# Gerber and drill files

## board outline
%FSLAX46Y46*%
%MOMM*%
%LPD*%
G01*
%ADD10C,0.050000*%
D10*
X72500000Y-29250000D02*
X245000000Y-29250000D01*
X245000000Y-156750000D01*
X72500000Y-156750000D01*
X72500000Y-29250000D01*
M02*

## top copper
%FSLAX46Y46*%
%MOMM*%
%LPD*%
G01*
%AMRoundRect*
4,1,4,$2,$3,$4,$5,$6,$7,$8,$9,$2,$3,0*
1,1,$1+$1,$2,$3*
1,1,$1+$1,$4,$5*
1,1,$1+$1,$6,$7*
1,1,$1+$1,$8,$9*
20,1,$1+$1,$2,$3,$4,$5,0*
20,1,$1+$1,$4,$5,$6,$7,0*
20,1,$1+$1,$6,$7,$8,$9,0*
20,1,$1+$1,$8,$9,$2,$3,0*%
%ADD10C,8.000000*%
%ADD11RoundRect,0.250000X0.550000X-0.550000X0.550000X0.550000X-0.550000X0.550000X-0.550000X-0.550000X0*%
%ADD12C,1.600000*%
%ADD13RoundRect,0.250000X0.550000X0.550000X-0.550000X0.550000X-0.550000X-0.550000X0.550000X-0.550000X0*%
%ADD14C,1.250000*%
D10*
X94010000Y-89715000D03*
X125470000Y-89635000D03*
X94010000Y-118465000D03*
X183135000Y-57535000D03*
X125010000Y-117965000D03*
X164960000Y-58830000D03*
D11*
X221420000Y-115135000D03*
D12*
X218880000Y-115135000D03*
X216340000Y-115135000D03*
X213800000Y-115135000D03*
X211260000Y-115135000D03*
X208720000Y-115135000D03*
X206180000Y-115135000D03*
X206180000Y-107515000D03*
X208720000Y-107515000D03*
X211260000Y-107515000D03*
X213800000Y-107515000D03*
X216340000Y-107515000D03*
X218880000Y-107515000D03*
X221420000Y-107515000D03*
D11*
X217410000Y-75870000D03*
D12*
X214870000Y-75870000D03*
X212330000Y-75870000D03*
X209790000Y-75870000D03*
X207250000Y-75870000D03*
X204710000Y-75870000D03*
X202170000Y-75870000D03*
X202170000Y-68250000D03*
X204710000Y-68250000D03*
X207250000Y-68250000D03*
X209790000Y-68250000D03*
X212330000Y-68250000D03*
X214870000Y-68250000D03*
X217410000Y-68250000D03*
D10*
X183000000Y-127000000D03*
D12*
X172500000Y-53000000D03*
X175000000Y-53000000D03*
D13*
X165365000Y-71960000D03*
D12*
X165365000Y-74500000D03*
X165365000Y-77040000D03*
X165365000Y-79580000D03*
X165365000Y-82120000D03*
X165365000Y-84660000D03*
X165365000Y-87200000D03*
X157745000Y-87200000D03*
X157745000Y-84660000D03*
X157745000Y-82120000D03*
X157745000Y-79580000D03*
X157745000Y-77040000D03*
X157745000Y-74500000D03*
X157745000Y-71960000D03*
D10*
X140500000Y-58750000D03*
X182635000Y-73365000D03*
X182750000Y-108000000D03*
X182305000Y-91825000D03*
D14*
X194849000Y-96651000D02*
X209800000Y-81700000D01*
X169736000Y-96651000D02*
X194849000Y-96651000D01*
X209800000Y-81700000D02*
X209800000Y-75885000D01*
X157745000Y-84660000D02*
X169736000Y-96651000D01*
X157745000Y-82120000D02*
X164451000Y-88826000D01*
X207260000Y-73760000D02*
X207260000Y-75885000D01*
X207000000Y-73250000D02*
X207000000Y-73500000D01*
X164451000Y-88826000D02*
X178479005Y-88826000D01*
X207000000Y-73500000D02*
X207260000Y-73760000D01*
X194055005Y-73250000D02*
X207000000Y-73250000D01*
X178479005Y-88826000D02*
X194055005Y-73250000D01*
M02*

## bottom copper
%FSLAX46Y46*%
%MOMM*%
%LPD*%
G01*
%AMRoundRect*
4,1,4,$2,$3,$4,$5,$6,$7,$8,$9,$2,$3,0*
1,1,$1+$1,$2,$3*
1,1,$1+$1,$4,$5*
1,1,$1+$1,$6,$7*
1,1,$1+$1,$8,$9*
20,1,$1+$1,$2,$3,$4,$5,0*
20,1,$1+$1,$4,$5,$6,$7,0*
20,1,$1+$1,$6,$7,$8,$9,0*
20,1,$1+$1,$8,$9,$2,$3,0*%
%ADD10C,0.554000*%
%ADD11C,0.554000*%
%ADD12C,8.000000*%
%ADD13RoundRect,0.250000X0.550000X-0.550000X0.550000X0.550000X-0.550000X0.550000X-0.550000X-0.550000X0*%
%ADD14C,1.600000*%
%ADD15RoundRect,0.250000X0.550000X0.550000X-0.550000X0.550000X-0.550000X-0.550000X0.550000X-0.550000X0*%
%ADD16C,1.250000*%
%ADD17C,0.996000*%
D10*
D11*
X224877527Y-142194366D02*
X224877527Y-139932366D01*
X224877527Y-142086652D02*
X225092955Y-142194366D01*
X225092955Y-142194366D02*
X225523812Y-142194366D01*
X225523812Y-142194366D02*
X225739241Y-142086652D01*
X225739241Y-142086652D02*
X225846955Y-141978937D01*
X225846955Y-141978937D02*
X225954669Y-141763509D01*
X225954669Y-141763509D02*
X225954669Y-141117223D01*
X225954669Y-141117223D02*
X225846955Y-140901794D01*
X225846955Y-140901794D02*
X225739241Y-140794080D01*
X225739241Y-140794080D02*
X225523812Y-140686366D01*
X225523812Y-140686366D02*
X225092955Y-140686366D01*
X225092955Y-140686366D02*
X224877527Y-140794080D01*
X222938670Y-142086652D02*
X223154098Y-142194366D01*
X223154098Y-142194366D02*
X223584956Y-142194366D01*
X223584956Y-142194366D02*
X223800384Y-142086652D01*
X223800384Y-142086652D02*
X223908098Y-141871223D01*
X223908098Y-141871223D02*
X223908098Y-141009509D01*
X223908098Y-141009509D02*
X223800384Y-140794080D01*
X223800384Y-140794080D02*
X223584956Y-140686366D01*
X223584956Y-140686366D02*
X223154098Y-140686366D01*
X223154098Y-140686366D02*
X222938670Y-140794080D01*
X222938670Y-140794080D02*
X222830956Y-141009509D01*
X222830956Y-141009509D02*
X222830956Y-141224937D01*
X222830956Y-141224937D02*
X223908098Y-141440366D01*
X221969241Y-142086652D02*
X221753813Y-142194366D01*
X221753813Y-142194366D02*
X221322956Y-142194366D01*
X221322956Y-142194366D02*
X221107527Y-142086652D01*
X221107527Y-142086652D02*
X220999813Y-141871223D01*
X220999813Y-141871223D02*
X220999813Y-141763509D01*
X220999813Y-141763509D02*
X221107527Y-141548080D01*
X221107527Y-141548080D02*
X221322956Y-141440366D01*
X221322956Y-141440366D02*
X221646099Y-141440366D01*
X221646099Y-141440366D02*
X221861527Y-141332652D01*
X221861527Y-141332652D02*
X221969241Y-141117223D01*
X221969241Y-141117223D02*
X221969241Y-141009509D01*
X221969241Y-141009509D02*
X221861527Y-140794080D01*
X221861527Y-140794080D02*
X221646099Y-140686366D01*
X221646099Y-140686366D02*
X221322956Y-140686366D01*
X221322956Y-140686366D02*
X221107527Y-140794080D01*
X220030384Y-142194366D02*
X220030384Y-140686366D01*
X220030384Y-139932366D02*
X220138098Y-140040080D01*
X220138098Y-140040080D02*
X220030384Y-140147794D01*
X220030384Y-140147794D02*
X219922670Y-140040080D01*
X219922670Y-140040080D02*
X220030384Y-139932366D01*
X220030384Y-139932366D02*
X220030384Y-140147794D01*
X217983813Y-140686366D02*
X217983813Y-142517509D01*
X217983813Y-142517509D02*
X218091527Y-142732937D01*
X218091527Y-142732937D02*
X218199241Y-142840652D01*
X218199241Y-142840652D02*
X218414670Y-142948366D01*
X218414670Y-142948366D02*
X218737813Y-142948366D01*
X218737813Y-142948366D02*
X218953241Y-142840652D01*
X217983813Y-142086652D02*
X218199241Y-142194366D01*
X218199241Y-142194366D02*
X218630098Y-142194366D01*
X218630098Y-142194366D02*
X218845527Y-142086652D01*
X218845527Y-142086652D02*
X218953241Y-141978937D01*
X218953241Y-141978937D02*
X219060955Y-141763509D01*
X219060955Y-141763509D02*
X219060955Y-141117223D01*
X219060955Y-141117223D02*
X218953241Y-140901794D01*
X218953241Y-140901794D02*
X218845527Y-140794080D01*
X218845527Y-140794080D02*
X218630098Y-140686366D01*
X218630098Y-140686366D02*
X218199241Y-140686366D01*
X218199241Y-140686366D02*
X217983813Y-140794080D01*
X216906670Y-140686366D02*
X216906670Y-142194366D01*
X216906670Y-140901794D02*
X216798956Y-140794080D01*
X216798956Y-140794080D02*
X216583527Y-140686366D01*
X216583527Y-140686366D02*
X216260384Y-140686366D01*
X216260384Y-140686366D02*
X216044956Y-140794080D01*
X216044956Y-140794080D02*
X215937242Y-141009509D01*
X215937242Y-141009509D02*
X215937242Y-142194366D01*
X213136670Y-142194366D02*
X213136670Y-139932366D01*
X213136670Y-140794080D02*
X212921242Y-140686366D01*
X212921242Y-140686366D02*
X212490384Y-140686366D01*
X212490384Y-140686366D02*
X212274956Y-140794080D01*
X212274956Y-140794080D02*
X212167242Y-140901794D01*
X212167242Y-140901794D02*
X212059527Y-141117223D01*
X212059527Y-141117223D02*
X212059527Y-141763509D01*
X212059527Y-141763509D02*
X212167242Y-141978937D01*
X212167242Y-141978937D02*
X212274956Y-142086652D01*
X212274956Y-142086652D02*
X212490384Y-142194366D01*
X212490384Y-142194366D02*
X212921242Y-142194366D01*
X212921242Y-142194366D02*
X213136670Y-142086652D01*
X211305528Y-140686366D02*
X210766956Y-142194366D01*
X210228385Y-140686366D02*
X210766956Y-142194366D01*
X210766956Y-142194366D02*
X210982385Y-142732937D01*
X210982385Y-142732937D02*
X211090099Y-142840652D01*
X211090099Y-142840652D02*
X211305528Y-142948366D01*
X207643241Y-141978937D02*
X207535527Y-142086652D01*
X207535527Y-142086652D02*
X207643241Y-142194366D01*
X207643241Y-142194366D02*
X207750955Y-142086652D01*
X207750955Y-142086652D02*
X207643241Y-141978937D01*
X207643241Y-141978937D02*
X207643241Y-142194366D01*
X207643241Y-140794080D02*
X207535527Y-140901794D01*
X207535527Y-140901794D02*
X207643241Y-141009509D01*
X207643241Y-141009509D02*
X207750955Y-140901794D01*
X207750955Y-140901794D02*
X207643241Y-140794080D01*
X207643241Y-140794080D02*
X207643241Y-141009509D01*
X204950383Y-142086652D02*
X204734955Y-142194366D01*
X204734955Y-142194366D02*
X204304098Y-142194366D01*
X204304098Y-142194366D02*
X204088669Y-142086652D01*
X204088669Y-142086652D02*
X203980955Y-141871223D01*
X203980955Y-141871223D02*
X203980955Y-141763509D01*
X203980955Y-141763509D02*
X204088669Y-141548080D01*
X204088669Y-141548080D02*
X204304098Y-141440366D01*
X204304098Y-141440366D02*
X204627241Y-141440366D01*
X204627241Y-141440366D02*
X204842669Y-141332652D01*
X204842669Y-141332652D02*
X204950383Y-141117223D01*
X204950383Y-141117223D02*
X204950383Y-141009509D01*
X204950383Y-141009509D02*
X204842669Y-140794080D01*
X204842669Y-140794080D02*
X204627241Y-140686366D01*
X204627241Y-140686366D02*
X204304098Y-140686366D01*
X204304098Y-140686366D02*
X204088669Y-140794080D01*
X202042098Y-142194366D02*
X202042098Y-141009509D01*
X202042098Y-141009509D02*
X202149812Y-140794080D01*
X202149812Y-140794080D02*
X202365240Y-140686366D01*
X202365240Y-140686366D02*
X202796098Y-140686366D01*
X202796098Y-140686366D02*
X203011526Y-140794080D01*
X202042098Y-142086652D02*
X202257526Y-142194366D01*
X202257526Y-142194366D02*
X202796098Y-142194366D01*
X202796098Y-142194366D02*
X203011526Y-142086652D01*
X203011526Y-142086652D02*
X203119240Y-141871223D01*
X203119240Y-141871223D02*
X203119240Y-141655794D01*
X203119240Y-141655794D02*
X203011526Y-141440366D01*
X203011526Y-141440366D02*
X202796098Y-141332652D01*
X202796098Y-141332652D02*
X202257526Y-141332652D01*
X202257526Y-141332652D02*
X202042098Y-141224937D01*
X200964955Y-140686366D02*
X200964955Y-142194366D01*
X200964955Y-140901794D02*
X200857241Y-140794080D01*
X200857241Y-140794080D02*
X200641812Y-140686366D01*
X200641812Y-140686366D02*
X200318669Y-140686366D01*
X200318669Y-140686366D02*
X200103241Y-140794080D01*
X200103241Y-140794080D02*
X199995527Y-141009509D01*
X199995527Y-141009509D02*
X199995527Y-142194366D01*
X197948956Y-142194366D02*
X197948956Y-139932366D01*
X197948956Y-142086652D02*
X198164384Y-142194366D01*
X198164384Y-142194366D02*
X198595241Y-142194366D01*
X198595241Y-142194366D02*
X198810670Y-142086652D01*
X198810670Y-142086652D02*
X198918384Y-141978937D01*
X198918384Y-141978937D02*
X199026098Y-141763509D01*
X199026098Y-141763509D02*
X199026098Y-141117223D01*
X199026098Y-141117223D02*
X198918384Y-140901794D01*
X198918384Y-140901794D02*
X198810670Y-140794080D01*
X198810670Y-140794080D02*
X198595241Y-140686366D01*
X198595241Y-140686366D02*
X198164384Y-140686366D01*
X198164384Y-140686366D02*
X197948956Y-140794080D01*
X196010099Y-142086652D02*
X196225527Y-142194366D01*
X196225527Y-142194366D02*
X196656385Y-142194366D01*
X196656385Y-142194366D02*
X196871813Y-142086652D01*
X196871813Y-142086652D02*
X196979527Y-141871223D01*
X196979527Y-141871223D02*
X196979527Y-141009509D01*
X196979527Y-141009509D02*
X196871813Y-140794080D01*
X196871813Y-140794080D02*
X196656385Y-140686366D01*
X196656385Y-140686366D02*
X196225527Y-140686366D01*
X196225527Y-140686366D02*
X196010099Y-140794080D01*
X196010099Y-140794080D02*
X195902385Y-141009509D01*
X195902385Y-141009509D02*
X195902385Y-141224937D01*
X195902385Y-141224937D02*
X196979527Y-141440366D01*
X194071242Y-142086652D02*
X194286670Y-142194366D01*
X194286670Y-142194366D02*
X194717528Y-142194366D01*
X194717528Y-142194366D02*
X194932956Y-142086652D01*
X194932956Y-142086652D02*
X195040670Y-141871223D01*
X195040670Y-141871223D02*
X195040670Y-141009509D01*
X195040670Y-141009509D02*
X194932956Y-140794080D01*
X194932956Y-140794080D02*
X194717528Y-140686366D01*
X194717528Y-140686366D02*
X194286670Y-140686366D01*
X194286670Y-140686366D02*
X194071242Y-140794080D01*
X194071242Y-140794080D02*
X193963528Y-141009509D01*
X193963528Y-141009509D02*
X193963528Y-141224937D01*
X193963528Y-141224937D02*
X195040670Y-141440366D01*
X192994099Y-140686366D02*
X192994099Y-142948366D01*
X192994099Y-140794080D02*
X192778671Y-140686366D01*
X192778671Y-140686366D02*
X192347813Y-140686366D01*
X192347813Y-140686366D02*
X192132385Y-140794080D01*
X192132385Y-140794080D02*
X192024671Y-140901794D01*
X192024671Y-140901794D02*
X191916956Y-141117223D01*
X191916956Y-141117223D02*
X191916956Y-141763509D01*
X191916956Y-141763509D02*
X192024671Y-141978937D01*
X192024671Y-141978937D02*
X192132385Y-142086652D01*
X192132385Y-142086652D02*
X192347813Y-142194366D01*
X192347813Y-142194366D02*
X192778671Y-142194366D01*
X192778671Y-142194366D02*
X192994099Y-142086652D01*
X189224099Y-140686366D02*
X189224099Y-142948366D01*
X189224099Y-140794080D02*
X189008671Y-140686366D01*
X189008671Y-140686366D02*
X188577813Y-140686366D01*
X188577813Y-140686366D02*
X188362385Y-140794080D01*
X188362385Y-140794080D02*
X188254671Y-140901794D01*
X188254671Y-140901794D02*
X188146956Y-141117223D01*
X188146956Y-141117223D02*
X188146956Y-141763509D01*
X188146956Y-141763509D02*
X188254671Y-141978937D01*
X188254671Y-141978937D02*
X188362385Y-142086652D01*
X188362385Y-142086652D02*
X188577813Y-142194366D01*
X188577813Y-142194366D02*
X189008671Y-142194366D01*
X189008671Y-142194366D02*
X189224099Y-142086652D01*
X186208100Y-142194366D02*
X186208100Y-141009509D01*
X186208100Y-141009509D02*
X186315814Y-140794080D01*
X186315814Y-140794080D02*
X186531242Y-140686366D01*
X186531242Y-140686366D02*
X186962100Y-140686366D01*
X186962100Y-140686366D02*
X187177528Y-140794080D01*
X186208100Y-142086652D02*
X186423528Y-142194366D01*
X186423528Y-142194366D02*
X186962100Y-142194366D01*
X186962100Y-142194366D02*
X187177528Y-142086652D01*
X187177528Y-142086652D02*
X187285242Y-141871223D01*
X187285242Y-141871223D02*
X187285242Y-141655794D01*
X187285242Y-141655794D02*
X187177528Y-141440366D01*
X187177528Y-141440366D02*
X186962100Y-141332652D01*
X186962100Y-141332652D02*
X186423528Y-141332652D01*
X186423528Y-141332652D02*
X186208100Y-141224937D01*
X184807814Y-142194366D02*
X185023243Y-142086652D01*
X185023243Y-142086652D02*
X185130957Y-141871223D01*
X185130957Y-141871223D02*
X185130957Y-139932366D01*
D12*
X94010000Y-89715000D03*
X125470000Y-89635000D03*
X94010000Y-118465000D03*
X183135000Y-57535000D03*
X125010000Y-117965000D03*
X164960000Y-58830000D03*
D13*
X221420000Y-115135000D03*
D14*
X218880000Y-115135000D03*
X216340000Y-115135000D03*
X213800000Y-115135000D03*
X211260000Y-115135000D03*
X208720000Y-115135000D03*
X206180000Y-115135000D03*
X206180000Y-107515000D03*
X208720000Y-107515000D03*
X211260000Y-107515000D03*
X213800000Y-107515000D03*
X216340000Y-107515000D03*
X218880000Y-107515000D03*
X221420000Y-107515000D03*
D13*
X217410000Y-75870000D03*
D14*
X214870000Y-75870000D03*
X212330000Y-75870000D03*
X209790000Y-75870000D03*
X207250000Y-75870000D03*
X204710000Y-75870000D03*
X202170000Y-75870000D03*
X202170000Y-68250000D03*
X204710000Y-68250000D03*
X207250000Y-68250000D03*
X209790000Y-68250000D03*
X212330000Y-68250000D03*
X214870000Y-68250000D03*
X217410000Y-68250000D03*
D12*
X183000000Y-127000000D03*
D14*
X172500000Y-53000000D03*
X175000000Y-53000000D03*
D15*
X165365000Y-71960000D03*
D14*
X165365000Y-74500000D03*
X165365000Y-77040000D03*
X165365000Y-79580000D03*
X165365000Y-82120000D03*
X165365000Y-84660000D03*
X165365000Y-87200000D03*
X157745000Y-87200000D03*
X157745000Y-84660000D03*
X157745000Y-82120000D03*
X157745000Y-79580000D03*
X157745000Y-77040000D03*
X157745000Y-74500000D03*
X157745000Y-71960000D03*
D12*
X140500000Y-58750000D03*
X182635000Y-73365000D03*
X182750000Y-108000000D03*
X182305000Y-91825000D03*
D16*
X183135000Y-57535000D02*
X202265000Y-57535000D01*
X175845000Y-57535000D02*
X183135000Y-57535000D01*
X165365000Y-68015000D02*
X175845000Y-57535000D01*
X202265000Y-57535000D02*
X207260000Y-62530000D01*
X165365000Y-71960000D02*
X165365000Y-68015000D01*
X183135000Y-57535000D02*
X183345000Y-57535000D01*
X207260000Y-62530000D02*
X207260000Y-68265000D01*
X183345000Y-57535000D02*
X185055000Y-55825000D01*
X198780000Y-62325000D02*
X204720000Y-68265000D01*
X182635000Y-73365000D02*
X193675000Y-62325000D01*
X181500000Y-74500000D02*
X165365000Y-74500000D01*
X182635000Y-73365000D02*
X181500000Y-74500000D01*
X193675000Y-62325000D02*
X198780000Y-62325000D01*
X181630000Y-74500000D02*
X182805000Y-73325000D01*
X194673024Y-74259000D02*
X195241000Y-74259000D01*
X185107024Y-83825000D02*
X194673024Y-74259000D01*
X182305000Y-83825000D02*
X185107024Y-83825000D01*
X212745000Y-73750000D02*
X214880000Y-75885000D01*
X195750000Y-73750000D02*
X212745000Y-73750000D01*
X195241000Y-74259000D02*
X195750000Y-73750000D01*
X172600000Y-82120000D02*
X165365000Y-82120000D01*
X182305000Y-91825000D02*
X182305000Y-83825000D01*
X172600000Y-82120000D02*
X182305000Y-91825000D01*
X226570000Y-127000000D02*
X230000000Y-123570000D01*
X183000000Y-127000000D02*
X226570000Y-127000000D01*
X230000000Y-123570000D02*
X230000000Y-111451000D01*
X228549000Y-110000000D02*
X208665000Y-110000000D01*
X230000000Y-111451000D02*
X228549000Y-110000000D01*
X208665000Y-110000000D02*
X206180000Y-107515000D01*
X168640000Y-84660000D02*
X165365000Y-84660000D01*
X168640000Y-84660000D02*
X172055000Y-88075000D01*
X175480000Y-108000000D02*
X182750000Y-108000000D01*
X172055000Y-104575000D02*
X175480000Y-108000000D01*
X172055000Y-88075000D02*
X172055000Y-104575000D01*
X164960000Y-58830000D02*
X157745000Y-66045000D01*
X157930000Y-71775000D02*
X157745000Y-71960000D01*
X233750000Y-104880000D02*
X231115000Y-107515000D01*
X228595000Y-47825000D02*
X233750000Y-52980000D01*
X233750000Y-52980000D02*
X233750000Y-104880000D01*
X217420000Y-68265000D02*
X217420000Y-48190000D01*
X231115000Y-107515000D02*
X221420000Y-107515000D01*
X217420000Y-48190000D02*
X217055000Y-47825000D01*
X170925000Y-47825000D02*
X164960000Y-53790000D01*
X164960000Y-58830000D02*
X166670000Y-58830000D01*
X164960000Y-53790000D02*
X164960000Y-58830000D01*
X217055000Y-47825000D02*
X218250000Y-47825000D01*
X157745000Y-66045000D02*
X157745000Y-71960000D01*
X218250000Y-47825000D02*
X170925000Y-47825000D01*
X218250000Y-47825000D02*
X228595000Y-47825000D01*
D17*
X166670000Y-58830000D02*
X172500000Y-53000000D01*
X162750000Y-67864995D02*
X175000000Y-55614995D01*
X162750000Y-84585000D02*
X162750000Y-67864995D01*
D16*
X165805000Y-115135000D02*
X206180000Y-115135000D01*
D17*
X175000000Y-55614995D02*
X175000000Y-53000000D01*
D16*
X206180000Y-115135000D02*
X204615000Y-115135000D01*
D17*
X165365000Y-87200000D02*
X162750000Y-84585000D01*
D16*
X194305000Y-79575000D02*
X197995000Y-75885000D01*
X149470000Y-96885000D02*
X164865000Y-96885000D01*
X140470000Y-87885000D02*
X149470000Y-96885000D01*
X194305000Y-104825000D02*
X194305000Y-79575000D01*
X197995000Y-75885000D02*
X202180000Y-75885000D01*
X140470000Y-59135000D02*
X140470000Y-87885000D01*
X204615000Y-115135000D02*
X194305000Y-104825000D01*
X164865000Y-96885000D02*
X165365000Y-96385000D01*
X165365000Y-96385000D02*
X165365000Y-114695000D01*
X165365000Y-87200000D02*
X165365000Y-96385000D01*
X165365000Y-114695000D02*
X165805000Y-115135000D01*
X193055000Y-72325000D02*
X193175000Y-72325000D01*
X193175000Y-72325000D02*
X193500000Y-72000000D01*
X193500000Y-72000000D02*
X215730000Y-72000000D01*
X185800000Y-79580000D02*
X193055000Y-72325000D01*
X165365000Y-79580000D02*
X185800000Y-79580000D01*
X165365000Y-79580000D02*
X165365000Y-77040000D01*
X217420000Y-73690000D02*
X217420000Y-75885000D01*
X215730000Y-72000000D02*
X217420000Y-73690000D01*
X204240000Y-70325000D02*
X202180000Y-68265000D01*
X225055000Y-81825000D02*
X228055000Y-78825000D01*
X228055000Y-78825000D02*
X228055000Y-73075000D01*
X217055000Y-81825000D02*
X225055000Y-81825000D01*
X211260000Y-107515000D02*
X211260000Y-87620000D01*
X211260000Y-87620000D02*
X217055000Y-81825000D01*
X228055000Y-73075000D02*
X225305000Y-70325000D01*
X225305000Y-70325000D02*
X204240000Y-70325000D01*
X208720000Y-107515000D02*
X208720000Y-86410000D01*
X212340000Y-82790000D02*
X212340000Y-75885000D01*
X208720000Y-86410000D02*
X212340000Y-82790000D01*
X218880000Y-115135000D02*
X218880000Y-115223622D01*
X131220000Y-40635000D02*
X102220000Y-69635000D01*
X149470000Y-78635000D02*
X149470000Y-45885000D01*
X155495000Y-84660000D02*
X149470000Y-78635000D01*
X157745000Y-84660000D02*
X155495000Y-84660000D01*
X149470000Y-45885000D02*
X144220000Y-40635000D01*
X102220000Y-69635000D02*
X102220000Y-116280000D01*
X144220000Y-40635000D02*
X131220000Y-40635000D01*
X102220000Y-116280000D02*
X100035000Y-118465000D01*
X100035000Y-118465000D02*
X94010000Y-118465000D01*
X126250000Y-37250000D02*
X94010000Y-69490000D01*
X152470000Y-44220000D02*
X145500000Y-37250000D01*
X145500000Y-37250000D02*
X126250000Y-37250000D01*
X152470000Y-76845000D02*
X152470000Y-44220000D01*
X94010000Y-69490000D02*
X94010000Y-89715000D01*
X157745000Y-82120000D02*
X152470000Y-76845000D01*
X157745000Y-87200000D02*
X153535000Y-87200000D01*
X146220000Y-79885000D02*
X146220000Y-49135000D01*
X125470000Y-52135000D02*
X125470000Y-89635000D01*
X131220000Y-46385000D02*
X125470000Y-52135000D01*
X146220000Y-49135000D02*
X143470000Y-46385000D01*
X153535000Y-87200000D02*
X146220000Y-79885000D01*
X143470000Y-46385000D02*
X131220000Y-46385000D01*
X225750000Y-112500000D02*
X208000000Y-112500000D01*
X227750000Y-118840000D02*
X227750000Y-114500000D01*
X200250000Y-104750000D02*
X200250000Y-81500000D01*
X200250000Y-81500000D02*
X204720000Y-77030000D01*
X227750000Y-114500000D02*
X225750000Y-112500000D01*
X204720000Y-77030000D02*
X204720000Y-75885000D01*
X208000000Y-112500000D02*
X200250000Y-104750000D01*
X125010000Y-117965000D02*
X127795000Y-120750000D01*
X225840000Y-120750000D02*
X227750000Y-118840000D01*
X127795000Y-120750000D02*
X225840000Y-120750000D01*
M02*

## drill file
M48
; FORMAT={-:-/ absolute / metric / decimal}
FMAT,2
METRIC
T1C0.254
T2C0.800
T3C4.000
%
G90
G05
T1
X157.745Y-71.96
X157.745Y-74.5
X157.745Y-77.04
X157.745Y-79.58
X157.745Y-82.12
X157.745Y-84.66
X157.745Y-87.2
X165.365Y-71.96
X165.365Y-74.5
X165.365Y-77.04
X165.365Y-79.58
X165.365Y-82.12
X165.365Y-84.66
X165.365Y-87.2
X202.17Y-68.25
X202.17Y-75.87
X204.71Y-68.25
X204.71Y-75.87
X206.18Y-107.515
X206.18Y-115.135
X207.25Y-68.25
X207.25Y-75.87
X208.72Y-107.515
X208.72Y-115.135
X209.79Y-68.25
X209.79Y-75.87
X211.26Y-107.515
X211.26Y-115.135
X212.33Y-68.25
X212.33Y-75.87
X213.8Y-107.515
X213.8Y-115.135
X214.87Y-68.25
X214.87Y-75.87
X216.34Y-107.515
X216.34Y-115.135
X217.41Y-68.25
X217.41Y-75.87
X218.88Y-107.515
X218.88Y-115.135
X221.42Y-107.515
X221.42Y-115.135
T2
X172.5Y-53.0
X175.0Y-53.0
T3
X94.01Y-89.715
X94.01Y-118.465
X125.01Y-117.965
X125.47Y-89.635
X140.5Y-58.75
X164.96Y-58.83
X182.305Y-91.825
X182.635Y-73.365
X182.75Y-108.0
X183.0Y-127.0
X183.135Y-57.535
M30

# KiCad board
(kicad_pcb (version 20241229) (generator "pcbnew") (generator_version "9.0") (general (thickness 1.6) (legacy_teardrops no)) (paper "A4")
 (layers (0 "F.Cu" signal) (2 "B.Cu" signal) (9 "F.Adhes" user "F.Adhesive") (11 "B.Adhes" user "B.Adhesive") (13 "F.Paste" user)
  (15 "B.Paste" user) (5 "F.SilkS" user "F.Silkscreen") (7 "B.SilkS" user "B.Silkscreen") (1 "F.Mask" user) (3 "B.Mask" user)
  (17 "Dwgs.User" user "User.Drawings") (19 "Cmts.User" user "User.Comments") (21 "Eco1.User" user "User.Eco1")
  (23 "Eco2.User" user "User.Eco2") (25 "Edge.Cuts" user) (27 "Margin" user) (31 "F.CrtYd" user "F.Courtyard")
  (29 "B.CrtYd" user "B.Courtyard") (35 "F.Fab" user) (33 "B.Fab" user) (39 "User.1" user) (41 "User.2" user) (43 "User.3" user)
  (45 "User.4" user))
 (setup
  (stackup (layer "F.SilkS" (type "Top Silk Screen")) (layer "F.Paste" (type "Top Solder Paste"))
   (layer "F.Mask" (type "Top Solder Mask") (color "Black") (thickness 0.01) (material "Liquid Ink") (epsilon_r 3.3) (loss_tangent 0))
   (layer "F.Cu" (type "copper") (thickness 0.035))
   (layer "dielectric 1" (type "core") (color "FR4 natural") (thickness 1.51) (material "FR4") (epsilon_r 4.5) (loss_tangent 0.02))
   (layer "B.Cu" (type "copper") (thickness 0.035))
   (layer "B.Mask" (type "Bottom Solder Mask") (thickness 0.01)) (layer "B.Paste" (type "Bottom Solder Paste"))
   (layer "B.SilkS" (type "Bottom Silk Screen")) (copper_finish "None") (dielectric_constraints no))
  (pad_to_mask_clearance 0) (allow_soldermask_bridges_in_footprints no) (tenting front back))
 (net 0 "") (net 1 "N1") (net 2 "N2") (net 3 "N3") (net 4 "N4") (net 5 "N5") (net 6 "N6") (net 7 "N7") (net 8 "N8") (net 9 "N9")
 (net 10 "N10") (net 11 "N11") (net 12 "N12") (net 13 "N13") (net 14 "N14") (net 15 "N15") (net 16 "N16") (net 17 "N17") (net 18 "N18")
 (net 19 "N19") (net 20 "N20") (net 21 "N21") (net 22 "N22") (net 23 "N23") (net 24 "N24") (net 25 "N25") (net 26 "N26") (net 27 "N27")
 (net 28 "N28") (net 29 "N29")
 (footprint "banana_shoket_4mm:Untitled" (layer "F.Cu") (at 94.22 89.635)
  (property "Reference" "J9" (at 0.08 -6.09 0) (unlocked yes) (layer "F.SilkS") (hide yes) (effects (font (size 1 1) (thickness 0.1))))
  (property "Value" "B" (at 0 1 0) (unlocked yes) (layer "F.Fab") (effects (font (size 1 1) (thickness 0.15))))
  (pad "1" thru_hole circle (at -0.21 0.08) (size 8 8) (drill 4) (layers "*.Cu" "*.Mask") (remove_unused_layers no) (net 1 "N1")))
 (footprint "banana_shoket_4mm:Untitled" (layer "F.Cu") (at 125.68 89.555)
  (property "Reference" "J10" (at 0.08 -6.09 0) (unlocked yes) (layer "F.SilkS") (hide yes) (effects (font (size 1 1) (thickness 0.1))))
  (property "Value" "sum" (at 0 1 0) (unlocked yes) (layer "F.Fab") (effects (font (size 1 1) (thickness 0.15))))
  (pad "1" thru_hole circle (at -0.21 0.08) (size 8 8) (drill 4) (layers "*.Cu" "*.Mask") (remove_unused_layers no) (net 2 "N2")))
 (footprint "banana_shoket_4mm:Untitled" (layer "F.Cu") (at 94.22 118.385)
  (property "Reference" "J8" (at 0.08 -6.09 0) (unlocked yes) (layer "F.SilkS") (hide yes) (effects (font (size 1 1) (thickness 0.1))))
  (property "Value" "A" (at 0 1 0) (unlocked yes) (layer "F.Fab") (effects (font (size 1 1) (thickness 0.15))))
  (pad "1" thru_hole circle (at -0.21 0.08) (size 8 8) (drill 4) (layers "*.Cu" "*.Mask") (remove_unused_layers no) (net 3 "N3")))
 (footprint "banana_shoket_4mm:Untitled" (layer "F.Cu") (at 183.055 57.325 90)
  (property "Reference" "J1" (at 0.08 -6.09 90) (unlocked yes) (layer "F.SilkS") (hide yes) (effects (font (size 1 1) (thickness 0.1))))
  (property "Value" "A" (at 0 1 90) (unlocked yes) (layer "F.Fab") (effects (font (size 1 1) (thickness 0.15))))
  (pad "1" thru_hole circle (at -0.21 0.08 90) (size 8 8) (drill 4) (layers "*.Cu" "*.Mask") (remove_unused_layers no) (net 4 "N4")))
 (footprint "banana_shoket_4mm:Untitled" (layer "F.Cu") (at 125.22 117.885)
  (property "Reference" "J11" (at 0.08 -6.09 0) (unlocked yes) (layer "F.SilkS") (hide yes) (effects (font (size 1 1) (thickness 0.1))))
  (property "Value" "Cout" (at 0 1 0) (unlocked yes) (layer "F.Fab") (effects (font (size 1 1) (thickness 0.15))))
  (pad "1" thru_hole circle (at -0.21 0.08) (size 8 8) (drill 4) (layers "*.Cu" "*.Mask") (remove_unused_layers no) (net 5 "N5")))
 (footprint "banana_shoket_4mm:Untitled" (layer "B.Cu") (at 164.75 58.75 180)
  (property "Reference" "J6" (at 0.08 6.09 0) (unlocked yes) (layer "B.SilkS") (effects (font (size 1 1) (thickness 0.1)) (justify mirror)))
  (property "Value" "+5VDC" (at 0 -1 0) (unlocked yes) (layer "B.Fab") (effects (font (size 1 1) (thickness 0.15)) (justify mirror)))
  (pad "1" thru_hole circle (at -0.21 -0.08 180) (size 8 8) (drill 4) (layers "*.Cu" "*.Mask") (remove_unused_layers no) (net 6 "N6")))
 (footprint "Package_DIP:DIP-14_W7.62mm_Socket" (layer "B.Cu") (at 221.42 115.135 90)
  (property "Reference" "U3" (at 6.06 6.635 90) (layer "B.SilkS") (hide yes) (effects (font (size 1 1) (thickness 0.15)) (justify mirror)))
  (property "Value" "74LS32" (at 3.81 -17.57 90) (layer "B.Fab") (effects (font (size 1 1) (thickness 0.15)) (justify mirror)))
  (pad "1" thru_hole roundrect (at 0 0 90) (size 1.6 1.6) (drill 0.254) (layers "*.Cu" "*.Mask") (remove_unused_layers no)
   (roundrect_rratio 0.15625) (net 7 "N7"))
  (pad "2" thru_hole circle (at 0 -2.54 90) (size 1.6 1.6) (drill 0.254) (layers "*.Cu" "*.Mask") (remove_unused_layers no) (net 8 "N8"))
  (pad "3" thru_hole circle (at 0 -5.08 90) (size 1.6 1.6) (drill 0.254) (layers "*.Cu" "*.Mask") (remove_unused_layers no) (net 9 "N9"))
  (pad "4" thru_hole circle (at 0 -7.62 90) (size 1.6 1.6) (drill 0.254) (layers "*.Cu" "*.Mask") (remove_unused_layers no) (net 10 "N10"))
  (pad "5" thru_hole circle (at 0 -10.16 90) (size 1.6 1.6) (drill 0.254) (layers "*.Cu" "*.Mask") (remove_unused_layers no) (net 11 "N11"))
  (pad "6" thru_hole circle (at 0 -12.7 90) (size 1.6 1.6) (drill 0.254) (layers "*.Cu" "*.Mask") (remove_unused_layers no) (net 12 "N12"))
  (pad "7" thru_hole circle (at 0 -15.24 90) (size 1.6 1.6) (drill 0.254) (layers "*.Cu" "*.Mask") (remove_unused_layers no) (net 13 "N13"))
  (pad "8" thru_hole circle (at 7.62 -15.24 90) (size 1.6 1.6) (drill 0.254) (layers "*.Cu" "*.Mask") (remove_unused_layers no)
   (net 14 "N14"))
  (pad "9" thru_hole circle (at 7.62 -12.7 90) (size 1.6 1.6) (drill 0.254) (layers "*.Cu" "*.Mask") (remove_unused_layers no)
   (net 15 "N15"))
  (pad "10" thru_hole circle (at 7.62 -10.16 90) (size 1.6 1.6) (drill 0.254) (layers "*.Cu" "*.Mask") (remove_unused_layers no)
   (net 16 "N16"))
  (pad "11" thru_hole circle (at 7.62 -7.62 90) (size 1.6 1.6) (drill 0.254) (layers "*.Cu" "*.Mask") (remove_unused_layers no)
   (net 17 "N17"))
  (pad "12" thru_hole circle (at 7.62 -5.08 90) (size 1.6 1.6) (drill 0.254) (layers "*.Cu" "*.Mask") (remove_unused_layers no)
   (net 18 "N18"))
  (pad "13" thru_hole circle (at 7.62 -2.54 90) (size 1.6 1.6) (drill 0.254) (layers "*.Cu" "*.Mask") (remove_unused_layers no)
   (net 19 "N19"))
  (pad "14" thru_hole circle (at 7.62 0 90) (size 1.6 1.6) (drill 0.254) (layers "*.Cu" "*.Mask") (remove_unused_layers no) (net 6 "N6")))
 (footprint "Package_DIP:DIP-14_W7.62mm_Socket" (layer "B.Cu") (at 217.41 75.87 90)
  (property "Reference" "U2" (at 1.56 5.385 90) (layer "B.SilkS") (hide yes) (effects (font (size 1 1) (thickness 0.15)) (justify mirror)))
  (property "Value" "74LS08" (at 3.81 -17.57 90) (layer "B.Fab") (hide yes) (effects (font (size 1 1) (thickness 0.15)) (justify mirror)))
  (pad "1" thru_hole roundrect (at 0 0 90) (size 1.6 1.6) (drill 0.254) (layers "*.Cu" "*.Mask") (remove_unused_layers no)
   (roundrect_rratio 0.15625) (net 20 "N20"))
  (pad "2" thru_hole circle (at 0 -2.54 90) (size 1.6 1.6) (drill 0.254) (layers "*.Cu" "*.Mask") (remove_unused_layers no) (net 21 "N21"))
  (pad "3" thru_hole circle (at 0 -5.08 90) (size 1.6 1.6) (drill 0.254) (layers "*.Cu" "*.Mask") (remove_unused_layers no) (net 15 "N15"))
  (pad "4" thru_hole circle (at 0 -7.62 90) (size 1.6 1.6) (drill 0.254) (layers "*.Cu" "*.Mask") (remove_unused_layers no) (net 3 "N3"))
  (pad "5" thru_hole circle (at 0 -10.16 90) (size 1.6 1.6) (drill 0.254) (layers "*.Cu" "*.Mask") (remove_unused_layers no) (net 1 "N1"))
  (pad "6" thru_hole circle (at 0 -12.7 90) (size 1.6 1.6) (drill 0.254) (layers "*.Cu" "*.Mask") (remove_unused_layers no) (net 5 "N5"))
  (pad "7" thru_hole circle (at 0 -15.24 90) (size 1.6 1.6) (drill 0.254) (layers "*.Cu" "*.Mask") (remove_unused_layers no) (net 13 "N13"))
  (pad "8" thru_hole circle (at 7.62 -15.24 90) (size 1.6 1.6) (drill 0.254) (layers "*.Cu" "*.Mask") (remove_unused_layers no)
   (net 16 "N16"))
  (pad "9" thru_hole circle (at 7.62 -12.7 90) (size 1.6 1.6) (drill 0.254) (layers "*.Cu" "*.Mask") (remove_unused_layers no)
   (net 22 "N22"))
  (pad "10" thru_hole circle (at 7.62 -10.16 90) (size 1.6 1.6) (drill 0.254) (layers "*.Cu" "*.Mask") (remove_unused_layers no)
   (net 4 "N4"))
  (pad "11" thru_hole circle (at 7.62 -7.62 90) (size 1.6 1.6) (drill 0.254) (layers "*.Cu" "*.Mask") (remove_unused_layers no)
   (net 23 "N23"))
  (pad "12" thru_hole circle (at 7.62 -5.08 90) (size 1.6 1.6) (drill 0.254) (layers "*.Cu" "*.Mask") (remove_unused_layers no)
   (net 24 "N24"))
  (pad "13" thru_hole circle (at 7.62 -2.54 90) (size 1.6 1.6) (drill 0.254) (layers "*.Cu" "*.Mask") (remove_unused_layers no)
   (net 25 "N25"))
  (pad "14" thru_hole circle (at 7.62 0 90) (size 1.6 1.6) (drill 0.254) (layers "*.Cu" "*.Mask") (remove_unused_layers no) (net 6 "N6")))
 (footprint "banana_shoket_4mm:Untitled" (layer "B.Cu") (at 182.79 126.92 180)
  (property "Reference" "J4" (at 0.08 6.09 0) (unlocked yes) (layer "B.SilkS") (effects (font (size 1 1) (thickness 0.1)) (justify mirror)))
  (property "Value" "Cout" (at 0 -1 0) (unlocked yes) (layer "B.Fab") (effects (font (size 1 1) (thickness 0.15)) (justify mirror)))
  (pad "1" thru_hole circle (at -0.21 -0.08 180) (size 8 8) (drill 4) (layers "*.Cu" "*.Mask") (remove_unused_layers no) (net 14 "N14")))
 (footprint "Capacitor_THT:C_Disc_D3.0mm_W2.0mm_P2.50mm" (layer "B.Cu") (at 172.5 53)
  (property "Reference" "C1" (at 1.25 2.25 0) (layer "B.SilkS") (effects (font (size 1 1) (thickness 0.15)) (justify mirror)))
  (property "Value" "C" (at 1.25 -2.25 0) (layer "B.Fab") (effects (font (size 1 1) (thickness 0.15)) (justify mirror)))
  (pad "1" thru_hole circle (at 0 0) (size 1.6 1.6) (drill 0.8) (layers "*.Cu" "*.Mask") (remove_unused_layers no) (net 6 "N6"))
  (pad "2" thru_hole circle (at 2.5 0) (size 1.6 1.6) (drill 0.8) (layers "*.Cu" "*.Mask") (remove_unused_layers no) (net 13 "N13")))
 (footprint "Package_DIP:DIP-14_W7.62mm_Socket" (layer "B.Cu") (at 165.365 71.96 180)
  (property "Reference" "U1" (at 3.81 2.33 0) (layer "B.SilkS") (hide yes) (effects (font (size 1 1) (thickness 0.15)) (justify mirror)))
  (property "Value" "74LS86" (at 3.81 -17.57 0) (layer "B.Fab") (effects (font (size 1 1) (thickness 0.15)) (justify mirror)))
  (pad "1" thru_hole roundrect (at 0 0 180) (size 1.6 1.6) (drill 0.254) (layers "*.Cu" "*.Mask") (remove_unused_layers no)
   (roundrect_rratio 0.15625) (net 4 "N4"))
  (pad "2" thru_hole circle (at 0 -2.54 180) (size 1.6 1.6) (drill 0.254) (layers "*.Cu" "*.Mask") (remove_unused_layers no) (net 22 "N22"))
  (pad "3" thru_hole circle (at 0 -5.08 180) (size 1.6 1.6) (drill 0.254) (layers "*.Cu" "*.Mask") (remove_unused_layers no) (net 20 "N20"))
  (pad "4" thru_hole circle (at 0 -7.62 180) (size 1.6 1.6) (drill 0.254) (layers "*.Cu" "*.Mask") (remove_unused_layers no) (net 20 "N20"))
  (pad "5" thru_hole circle (at 0 -10.16 180) (size 1.6 1.6) (drill 0.254) (layers "*.Cu" "*.Mask") (remove_unused_layers no) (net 21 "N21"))
  (pad "6" thru_hole circle (at 0 -12.7 180) (size 1.6 1.6) (drill 0.254) (layers "*.Cu" "*.Mask") (remove_unused_layers no) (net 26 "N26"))
  (pad "7" thru_hole circle (at 0 -15.24 180) (size 1.6 1.6) (drill 0.254) (layers "*.Cu" "*.Mask") (remove_unused_layers no) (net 13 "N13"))
  (pad "8" thru_hole circle (at 7.62 -15.24 180) (size 1.6 1.6) (drill 0.254) (layers "*.Cu" "*.Mask") (remove_unused_layers no)
   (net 2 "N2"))
  (pad "9" thru_hole circle (at 7.62 -12.7 180) (size 1.6 1.6) (drill 0.254) (layers "*.Cu" "*.Mask") (remove_unused_layers no) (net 3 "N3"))
  (pad "10" thru_hole circle (at 7.62 -10.16 180) (size 1.6 1.6) (drill 0.254) (layers "*.Cu" "*.Mask") (remove_unused_layers no)
   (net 1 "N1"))
  (pad "11" thru_hole circle (at 7.62 -7.62 180) (size 1.6 1.6) (drill 0.254) (layers "*.Cu" "*.Mask") (remove_unused_layers no)
   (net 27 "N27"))
  (pad "12" thru_hole circle (at 7.62 -5.08 180) (size 1.6 1.6) (drill 0.254) (layers "*.Cu" "*.Mask") (remove_unused_layers no)
   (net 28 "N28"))
  (pad "13" thru_hole circle (at 7.62 -2.54 180) (size 1.6 1.6) (drill 0.254) (layers "*.Cu" "*.Mask") (remove_unused_layers no)
   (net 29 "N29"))
  (pad "14" thru_hole circle (at 7.62 0 180) (size 1.6 1.6) (drill 0.254) (layers "*.Cu" "*.Mask") (remove_unused_layers no) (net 6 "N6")))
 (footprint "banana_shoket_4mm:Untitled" (layer "B.Cu") (at 140.42 58.96 -90)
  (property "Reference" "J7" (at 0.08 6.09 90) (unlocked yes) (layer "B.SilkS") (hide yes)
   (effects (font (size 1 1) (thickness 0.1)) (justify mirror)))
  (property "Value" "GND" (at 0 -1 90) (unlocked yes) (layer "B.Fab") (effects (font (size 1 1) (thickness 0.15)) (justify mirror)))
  (pad "1" thru_hole circle (at -0.21 -0.08 270) (size 8 8) (drill 4) (layers "*.Cu" "*.Mask") (remove_unused_layers no) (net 13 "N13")))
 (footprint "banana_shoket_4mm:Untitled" (layer "B.Cu") (at 182.555 73.575 -90)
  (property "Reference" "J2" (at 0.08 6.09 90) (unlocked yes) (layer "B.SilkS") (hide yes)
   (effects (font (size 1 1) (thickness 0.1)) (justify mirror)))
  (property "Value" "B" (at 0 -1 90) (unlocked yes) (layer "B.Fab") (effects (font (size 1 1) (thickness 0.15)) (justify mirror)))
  (pad "1" thru_hole circle (at -0.21 -0.08 270) (size 8 8) (drill 4) (layers "*.Cu" "*.Mask") (remove_unused_layers no) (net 22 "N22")))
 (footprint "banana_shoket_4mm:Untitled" (layer "B.Cu") (at 182.54 107.92 180)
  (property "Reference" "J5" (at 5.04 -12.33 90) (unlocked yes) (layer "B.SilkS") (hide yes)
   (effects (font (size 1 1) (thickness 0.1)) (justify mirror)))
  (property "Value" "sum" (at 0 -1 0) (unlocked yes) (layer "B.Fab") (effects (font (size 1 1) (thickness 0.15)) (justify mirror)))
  (pad "1" thru_hole circle (at -0.21 -0.08 180) (size 8 8) (drill 4) (layers "*.Cu" "*.Mask") (remove_unused_layers no) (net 26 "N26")))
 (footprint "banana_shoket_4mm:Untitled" (layer "B.Cu") (at 182.225 92.035 -90)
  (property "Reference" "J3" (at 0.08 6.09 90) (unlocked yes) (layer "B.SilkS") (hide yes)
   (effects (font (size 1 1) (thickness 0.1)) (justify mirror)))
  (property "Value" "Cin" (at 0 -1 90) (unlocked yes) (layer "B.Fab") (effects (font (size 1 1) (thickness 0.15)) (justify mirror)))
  (pad "1" thru_hole circle (at -0.21 -0.08 270) (size 8 8) (drill 4) (layers "*.Cu" "*.Mask") (remove_unused_layers no) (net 21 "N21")))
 (gr_rect (start 72.5 29.25) (end 245 156.75) (stroke (width 0.05) (type default)) (fill no) (layer "Edge.Cuts"))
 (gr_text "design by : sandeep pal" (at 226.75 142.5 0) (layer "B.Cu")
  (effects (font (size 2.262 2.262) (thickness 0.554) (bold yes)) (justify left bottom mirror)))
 (segment (start 183.135 57.535) (end 202.265 57.535) (width 1.25) (layer "B.Cu") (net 4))
 (segment (start 175.845 57.535) (end 183.135 57.535) (width 1.25) (layer "B.Cu") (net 4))
 (segment (start 165.365 68.015) (end 175.845 57.535) (width 1.25) (layer "B.Cu") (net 4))
 (segment (start 202.265 57.535) (end 207.26 62.53) (width 1.25) (layer "B.Cu") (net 4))
 (segment (start 165.365 71.96) (end 165.365 68.015) (width 1.25) (layer "B.Cu") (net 4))
 (segment (start 183.135 57.535) (end 183.345 57.535) (width 1.25) (layer "B.Cu") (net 4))
 (segment (start 207.26 62.53) (end 207.26 68.265) (width 1.25) (layer "B.Cu") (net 4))
 (segment (start 183.345 57.535) (end 185.055 55.825) (width 1.25) (layer "B.Cu") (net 4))
 (segment (start 198.78 62.325) (end 204.72 68.265) (width 1.25) (layer "B.Cu") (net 22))
 (segment (start 182.635 73.365) (end 193.675 62.325) (width 1.25) (layer "B.Cu") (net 22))
 (segment (start 181.5 74.5) (end 165.365 74.5) (width 1.25) (layer "B.Cu") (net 22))
 (segment (start 182.635 73.365) (end 181.5 74.5) (width 1.25) (layer "B.Cu") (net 22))
 (segment (start 193.675 62.325) (end 198.78 62.325) (width 1.25) (layer "B.Cu") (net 22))
 (segment (start 181.63 74.5) (end 182.805 73.325) (width 1.25) (layer "B.Cu") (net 22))
 (segment (start 194.673024 74.259) (end 195.241 74.259) (width 1.25) (layer "B.Cu") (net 21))
 (segment (start 185.107024 83.825) (end 194.673024 74.259) (width 1.25) (layer "B.Cu") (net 21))
 (segment (start 182.305 83.825) (end 185.107024 83.825) (width 1.25) (layer "B.Cu") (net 21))
 (segment (start 212.745 73.75) (end 214.88 75.885) (width 1.25) (layer "B.Cu") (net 21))
 (segment (start 195.75 73.75) (end 212.745 73.75) (width 1.25) (layer "B.Cu") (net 21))
 (segment (start 195.241 74.259) (end 195.75 73.75) (width 1.25) (layer "B.Cu") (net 21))
 (segment (start 172.6 82.12) (end 165.365 82.12) (width 1.25) (layer "B.Cu") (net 21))
 (segment (start 182.305 91.825) (end 182.305 83.825) (width 1.25) (layer "B.Cu") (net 21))
 (segment (start 172.6 82.12) (end 182.305 91.825) (width 1.25) (layer "B.Cu") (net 21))
 (segment (start 226.57 127) (end 230 123.57) (width 1.25) (layer "B.Cu") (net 14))
 (segment (start 183 127) (end 226.57 127) (width 1.25) (layer "B.Cu") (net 14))
 (segment (start 230 123.57) (end 230 111.451) (width 1.25) (layer "B.Cu") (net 14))
 (segment (start 228.549 110) (end 208.665 110) (width 1.25) (layer "B.Cu") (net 14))
 (segment (start 230 111.451) (end 228.549 110) (width 1.25) (layer "B.Cu") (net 14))
 (segment (start 208.665 110) (end 206.18 107.515) (width 1.25) (layer "B.Cu") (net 14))
 (segment (start 168.64 84.66) (end 165.365 84.66) (width 1.25) (layer "B.Cu") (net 26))
 (segment (start 168.64 84.66) (end 172.055 88.075) (width 1.25) (layer "B.Cu") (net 26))
 (segment (start 175.48 108) (end 182.75 108) (width 1.25) (layer "B.Cu") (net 26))
 (segment (start 172.055 104.575) (end 175.48 108) (width 1.25) (layer "B.Cu") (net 26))
 (segment (start 172.055 88.075) (end 172.055 104.575) (width 1.25) (layer "B.Cu") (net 26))
 (segment (start 164.96 58.83) (end 157.745 66.045) (width 1.25) (layer "B.Cu") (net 6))
 (segment (start 157.93 71.775) (end 157.745 71.96) (width 1.25) (layer "B.Cu") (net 6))
 (segment (start 233.75 104.88) (end 231.115 107.515) (width 1.25) (layer "B.Cu") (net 6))
 (segment (start 228.595 47.825) (end 233.75 52.98) (width 1.25) (layer "B.Cu") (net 6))
 (segment (start 233.75 52.98) (end 233.75 104.88) (width 1.25) (layer "B.Cu") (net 6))
 (segment (start 217.42 68.265) (end 217.42 48.19) (width 1.25) (layer "B.Cu") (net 6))
 (segment (start 231.115 107.515) (end 221.42 107.515) (width 1.25) (layer "B.Cu") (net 6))
 (segment (start 217.42 48.19) (end 217.055 47.825) (width 1.25) (layer "B.Cu") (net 6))
 (segment (start 170.925 47.825) (end 164.96 53.79) (width 1.25) (layer "B.Cu") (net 6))
 (segment (start 164.96 58.83) (end 166.67 58.83) (width 1.25) (layer "B.Cu") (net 6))
 (segment (start 164.96 53.79) (end 164.96 58.83) (width 1.25) (layer "B.Cu") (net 6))
 (segment (start 217.055 47.825) (end 218.25 47.825) (width 1.25) (layer "B.Cu") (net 6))
 (segment (start 157.745 66.045) (end 157.745 71.96) (width 1.25) (layer "B.Cu") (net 6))
 (segment (start 218.25 47.825) (end 170.925 47.825) (width 1.25) (layer "B.Cu") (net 6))
 (segment (start 218.25 47.825) (end 228.595 47.825) (width 1.25) (layer "B.Cu") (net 6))
 (segment (start 166.67 58.83) (end 172.5 53) (width 0.996) (layer "B.Cu") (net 6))
 (segment (start 162.75 67.864995) (end 175 55.614995) (width 0.996) (layer "B.Cu") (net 13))
 (segment (start 162.75 84.585) (end 162.75 67.864995) (width 0.996) (layer "B.Cu") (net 13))
 (segment (start 165.805 115.135) (end 206.18 115.135) (width 1.25) (layer "B.Cu") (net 13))
 (segment (start 175 55.614995) (end 175 53) (width 0.996) (layer "B.Cu") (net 13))
 (segment (start 206.18 115.135) (end 204.615 115.135) (width 1.25) (layer "B.Cu") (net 13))
 (segment (start 165.365 87.2) (end 162.75 84.585) (width 0.996) (layer "B.Cu") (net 13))
 (segment (start 194.305 79.575) (end 197.995 75.885) (width 1.25) (layer "B.Cu") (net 13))
 (segment (start 149.47 96.885) (end 164.865 96.885) (width 1.25) (layer "B.Cu") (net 13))
 (segment (start 140.47 87.885) (end 149.47 96.885) (width 1.25) (layer "B.Cu") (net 13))
 (segment (start 194.305 104.825) (end 194.305 79.575) (width 1.25) (layer "B.Cu") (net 13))
 (segment (start 197.995 75.885) (end 202.18 75.885) (width 1.25) (layer "B.Cu") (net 13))
 (segment (start 140.47 59.135) (end 140.47 87.885) (width 1.25) (layer "B.Cu") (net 13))
 (segment (start 204.615 115.135) (end 194.305 104.825) (width 1.25) (layer "B.Cu") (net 13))
 (segment (start 164.865 96.885) (end 165.365 96.385) (width 1.25) (layer "B.Cu") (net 13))
 (segment (start 165.365 96.385) (end 165.365 114.695) (width 1.25) (layer "B.Cu") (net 13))
 (segment (start 165.365 87.2) (end 165.365 96.385) (width 1.25) (layer "B.Cu") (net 13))
 (segment (start 165.365 114.695) (end 165.805 115.135) (width 1.25) (layer "B.Cu") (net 13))
 (segment (start 193.055 72.325) (end 193.175 72.325) (width 1.25) (layer "B.Cu") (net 20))
 (segment (start 193.175 72.325) (end 193.5 72) (width 1.25) (layer "B.Cu") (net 20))
 (segment (start 193.5 72) (end 215.73 72) (width 1.25) (layer "B.Cu") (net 20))
 (segment (start 185.8 79.58) (end 193.055 72.325) (width 1.25) (layer "B.Cu") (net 20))
 (segment (start 165.365 79.58) (end 185.8 79.58) (width 1.25) (layer "B.Cu") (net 20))
 (segment (start 165.365 79.58) (end 165.365 77.04) (width 1.25) (layer "B.Cu") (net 20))
 (segment (start 217.42 73.69) (end 217.42 75.885) (width 1.25) (layer "B.Cu") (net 20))
 (segment (start 215.73 72) (end 217.42 73.69) (width 1.25) (layer "B.Cu") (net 20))
 (segment (start 204.24 70.325) (end 202.18 68.265) (width 1.25) (layer "B.Cu") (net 16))
 (segment (start 225.055 81.825) (end 228.055 78.825) (width 1.25) (layer "B.Cu") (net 16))
 (segment (start 228.055 78.825) (end 228.055 73.075) (width 1.25) (layer "B.Cu") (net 16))
 (segment (start 217.055 81.825) (end 225.055 81.825) (width 1.25) (layer "B.Cu") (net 16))
 (segment (start 211.26 107.515) (end 211.26 87.62) (width 1.25) (layer "B.Cu") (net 16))
 (segment (start 211.26 87.62) (end 217.055 81.825) (width 1.25) (layer "B.Cu") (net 16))
 (segment (start 228.055 73.075) (end 225.305 70.325) (width 1.25) (layer "B.Cu") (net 16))
 (segment (start 225.305 70.325) (end 204.24 70.325) (width 1.25) (layer "B.Cu") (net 16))
 (segment (start 208.72 107.515) (end 208.72 86.41) (width 1.25) (layer "B.Cu") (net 15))
 (segment (start 212.34 82.79) (end 212.34 75.885) (width 1.25) (layer "B.Cu") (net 15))
 (segment (start 208.72 86.41) (end 212.34 82.79) (width 1.25) (layer "B.Cu") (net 15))
 (segment (start 218.88 115.135) (end 218.88 115.223622) (width 1.25) (layer "B.Cu") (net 8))
 (segment (start 194.849 96.651) (end 209.8 81.7) (width 1.25) (layer "F.Cu") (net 3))
 (segment (start 169.736 96.651) (end 194.849 96.651) (width 1.25) (layer "F.Cu") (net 3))
 (segment (start 209.8 81.7) (end 209.8 75.885) (width 1.25) (layer "F.Cu") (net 3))
 (segment (start 157.745 84.66) (end 169.736 96.651) (width 1.25) (layer "F.Cu") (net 3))
 (segment (start 131.22 40.635) (end 102.22 69.635) (width 1.25) (layer "B.Cu") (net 3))
 (segment (start 149.47 78.635) (end 149.47 45.885) (width 1.25) (layer "B.Cu") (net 3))
 (segment (start 155.495 84.66) (end 149.47 78.635) (width 1.25) (layer "B.Cu") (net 3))
 (segment (start 157.745 84.66) (end 155.495 84.66) (width 1.25) (layer "B.Cu") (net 3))
 (segment (start 149.47 45.885) (end 144.22 40.635) (width 1.25) (layer "B.Cu") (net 3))
 (segment (start 102.22 69.635) (end 102.22 116.28) (width 1.25) (layer "B.Cu") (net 3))
 (segment (start 144.22 40.635) (end 131.22 40.635) (width 1.25) (layer "B.Cu") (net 3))
 (segment (start 102.22 116.28) (end 100.035 118.465) (width 1.25) (layer "B.Cu") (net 3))
 (segment (start 100.035 118.465) (end 94.01 118.465) (width 1.25) (layer "B.Cu") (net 3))
 (segment (start 157.745 82.12) (end 164.451 88.826) (width 1.25) (layer "F.Cu") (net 1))
 (segment (start 207.26 73.76) (end 207.26 75.885) (width 1.25) (layer "F.Cu") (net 1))
 (segment (start 207 73.25) (end 207 73.5) (width 1.25) (layer "F.Cu") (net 1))
 (segment (start 164.451 88.826) (end 178.479005 88.826) (width 1.25) (layer "F.Cu") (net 1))
 (segment (start 207 73.5) (end 207.26 73.76) (width 1.25) (layer "F.Cu") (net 1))
 (segment (start 194.055005 73.25) (end 207 73.25) (width 1.25) (layer "F.Cu") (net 1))
 (segment (start 178.479005 88.826) (end 194.055005 73.25) (width 1.25) (layer "F.Cu") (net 1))
 (segment (start 126.25 37.25) (end 94.01 69.49) (width 1.25) (layer "B.Cu") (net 1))
 (segment (start 152.47 44.22) (end 145.5 37.25) (width 1.25) (layer "B.Cu") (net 1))
 (segment (start 145.5 37.25) (end 126.25 37.25) (width 1.25) (layer "B.Cu") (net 1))
 (segment (start 152.47 76.845) (end 152.47 44.22) (width 1.25) (layer "B.Cu") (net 1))
 (segment (start 94.01 69.49) (end 94.01 89.715) (width 1.25) (layer "B.Cu") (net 1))
 (segment (start 157.745 82.12) (end 152.47 76.845) (width 1.25) (layer "B.Cu") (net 1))
 (segment (start 157.745 87.2) (end 153.535 87.2) (width 1.25) (layer "B.Cu") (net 2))
 (segment (start 146.22 79.885) (end 146.22 49.135) (width 1.25) (layer "B.Cu") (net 2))
 (segment (start 125.47 52.135) (end 125.47 89.635) (width 1.25) (layer "B.Cu") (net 2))
 (segment (start 131.22 46.385) (end 125.47 52.135) (width 1.25) (layer "B.Cu") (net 2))
 (segment (start 146.22 49.135) (end 143.47 46.385) (width 1.25) (layer "B.Cu") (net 2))
 (segment (start 153.535 87.2) (end 146.22 79.885) (width 1.25) (layer "B.Cu") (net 2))
 (segment (start 143.47 46.385) (end 131.22 46.385) (width 1.25) (layer "B.Cu") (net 2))
 (segment (start 225.75 112.5) (end 208 112.5) (width 1.25) (layer "B.Cu") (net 5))
 (segment (start 227.75 118.84) (end 227.75 114.5) (width 1.25) (layer "B.Cu") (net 5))
 (segment (start 200.25 104.75) (end 200.25 81.5) (width 1.25) (layer "B.Cu") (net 5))
 (segment (start 200.25 81.5) (end 204.72 77.03) (width 1.25) (layer "B.Cu") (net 5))
 (segment (start 227.75 114.5) (end 225.75 112.5) (width 1.25) (layer "B.Cu") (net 5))
 (segment (start 204.72 77.03) (end 204.72 75.885) (width 1.25) (layer "B.Cu") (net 5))
 (segment (start 208 112.5) (end 200.25 104.75) (width 1.25) (layer "B.Cu") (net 5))
 (segment (start 125.01 117.965) (end 127.795 120.75) (width 1.25) (layer "B.Cu") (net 5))
 (segment (start 225.84 120.75) (end 227.75 118.84) (width 1.25) (layer "B.Cu") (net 5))
 (segment (start 127.795 120.75) (end 225.84 120.75) (width 1.25) (layer "B.Cu") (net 5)))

